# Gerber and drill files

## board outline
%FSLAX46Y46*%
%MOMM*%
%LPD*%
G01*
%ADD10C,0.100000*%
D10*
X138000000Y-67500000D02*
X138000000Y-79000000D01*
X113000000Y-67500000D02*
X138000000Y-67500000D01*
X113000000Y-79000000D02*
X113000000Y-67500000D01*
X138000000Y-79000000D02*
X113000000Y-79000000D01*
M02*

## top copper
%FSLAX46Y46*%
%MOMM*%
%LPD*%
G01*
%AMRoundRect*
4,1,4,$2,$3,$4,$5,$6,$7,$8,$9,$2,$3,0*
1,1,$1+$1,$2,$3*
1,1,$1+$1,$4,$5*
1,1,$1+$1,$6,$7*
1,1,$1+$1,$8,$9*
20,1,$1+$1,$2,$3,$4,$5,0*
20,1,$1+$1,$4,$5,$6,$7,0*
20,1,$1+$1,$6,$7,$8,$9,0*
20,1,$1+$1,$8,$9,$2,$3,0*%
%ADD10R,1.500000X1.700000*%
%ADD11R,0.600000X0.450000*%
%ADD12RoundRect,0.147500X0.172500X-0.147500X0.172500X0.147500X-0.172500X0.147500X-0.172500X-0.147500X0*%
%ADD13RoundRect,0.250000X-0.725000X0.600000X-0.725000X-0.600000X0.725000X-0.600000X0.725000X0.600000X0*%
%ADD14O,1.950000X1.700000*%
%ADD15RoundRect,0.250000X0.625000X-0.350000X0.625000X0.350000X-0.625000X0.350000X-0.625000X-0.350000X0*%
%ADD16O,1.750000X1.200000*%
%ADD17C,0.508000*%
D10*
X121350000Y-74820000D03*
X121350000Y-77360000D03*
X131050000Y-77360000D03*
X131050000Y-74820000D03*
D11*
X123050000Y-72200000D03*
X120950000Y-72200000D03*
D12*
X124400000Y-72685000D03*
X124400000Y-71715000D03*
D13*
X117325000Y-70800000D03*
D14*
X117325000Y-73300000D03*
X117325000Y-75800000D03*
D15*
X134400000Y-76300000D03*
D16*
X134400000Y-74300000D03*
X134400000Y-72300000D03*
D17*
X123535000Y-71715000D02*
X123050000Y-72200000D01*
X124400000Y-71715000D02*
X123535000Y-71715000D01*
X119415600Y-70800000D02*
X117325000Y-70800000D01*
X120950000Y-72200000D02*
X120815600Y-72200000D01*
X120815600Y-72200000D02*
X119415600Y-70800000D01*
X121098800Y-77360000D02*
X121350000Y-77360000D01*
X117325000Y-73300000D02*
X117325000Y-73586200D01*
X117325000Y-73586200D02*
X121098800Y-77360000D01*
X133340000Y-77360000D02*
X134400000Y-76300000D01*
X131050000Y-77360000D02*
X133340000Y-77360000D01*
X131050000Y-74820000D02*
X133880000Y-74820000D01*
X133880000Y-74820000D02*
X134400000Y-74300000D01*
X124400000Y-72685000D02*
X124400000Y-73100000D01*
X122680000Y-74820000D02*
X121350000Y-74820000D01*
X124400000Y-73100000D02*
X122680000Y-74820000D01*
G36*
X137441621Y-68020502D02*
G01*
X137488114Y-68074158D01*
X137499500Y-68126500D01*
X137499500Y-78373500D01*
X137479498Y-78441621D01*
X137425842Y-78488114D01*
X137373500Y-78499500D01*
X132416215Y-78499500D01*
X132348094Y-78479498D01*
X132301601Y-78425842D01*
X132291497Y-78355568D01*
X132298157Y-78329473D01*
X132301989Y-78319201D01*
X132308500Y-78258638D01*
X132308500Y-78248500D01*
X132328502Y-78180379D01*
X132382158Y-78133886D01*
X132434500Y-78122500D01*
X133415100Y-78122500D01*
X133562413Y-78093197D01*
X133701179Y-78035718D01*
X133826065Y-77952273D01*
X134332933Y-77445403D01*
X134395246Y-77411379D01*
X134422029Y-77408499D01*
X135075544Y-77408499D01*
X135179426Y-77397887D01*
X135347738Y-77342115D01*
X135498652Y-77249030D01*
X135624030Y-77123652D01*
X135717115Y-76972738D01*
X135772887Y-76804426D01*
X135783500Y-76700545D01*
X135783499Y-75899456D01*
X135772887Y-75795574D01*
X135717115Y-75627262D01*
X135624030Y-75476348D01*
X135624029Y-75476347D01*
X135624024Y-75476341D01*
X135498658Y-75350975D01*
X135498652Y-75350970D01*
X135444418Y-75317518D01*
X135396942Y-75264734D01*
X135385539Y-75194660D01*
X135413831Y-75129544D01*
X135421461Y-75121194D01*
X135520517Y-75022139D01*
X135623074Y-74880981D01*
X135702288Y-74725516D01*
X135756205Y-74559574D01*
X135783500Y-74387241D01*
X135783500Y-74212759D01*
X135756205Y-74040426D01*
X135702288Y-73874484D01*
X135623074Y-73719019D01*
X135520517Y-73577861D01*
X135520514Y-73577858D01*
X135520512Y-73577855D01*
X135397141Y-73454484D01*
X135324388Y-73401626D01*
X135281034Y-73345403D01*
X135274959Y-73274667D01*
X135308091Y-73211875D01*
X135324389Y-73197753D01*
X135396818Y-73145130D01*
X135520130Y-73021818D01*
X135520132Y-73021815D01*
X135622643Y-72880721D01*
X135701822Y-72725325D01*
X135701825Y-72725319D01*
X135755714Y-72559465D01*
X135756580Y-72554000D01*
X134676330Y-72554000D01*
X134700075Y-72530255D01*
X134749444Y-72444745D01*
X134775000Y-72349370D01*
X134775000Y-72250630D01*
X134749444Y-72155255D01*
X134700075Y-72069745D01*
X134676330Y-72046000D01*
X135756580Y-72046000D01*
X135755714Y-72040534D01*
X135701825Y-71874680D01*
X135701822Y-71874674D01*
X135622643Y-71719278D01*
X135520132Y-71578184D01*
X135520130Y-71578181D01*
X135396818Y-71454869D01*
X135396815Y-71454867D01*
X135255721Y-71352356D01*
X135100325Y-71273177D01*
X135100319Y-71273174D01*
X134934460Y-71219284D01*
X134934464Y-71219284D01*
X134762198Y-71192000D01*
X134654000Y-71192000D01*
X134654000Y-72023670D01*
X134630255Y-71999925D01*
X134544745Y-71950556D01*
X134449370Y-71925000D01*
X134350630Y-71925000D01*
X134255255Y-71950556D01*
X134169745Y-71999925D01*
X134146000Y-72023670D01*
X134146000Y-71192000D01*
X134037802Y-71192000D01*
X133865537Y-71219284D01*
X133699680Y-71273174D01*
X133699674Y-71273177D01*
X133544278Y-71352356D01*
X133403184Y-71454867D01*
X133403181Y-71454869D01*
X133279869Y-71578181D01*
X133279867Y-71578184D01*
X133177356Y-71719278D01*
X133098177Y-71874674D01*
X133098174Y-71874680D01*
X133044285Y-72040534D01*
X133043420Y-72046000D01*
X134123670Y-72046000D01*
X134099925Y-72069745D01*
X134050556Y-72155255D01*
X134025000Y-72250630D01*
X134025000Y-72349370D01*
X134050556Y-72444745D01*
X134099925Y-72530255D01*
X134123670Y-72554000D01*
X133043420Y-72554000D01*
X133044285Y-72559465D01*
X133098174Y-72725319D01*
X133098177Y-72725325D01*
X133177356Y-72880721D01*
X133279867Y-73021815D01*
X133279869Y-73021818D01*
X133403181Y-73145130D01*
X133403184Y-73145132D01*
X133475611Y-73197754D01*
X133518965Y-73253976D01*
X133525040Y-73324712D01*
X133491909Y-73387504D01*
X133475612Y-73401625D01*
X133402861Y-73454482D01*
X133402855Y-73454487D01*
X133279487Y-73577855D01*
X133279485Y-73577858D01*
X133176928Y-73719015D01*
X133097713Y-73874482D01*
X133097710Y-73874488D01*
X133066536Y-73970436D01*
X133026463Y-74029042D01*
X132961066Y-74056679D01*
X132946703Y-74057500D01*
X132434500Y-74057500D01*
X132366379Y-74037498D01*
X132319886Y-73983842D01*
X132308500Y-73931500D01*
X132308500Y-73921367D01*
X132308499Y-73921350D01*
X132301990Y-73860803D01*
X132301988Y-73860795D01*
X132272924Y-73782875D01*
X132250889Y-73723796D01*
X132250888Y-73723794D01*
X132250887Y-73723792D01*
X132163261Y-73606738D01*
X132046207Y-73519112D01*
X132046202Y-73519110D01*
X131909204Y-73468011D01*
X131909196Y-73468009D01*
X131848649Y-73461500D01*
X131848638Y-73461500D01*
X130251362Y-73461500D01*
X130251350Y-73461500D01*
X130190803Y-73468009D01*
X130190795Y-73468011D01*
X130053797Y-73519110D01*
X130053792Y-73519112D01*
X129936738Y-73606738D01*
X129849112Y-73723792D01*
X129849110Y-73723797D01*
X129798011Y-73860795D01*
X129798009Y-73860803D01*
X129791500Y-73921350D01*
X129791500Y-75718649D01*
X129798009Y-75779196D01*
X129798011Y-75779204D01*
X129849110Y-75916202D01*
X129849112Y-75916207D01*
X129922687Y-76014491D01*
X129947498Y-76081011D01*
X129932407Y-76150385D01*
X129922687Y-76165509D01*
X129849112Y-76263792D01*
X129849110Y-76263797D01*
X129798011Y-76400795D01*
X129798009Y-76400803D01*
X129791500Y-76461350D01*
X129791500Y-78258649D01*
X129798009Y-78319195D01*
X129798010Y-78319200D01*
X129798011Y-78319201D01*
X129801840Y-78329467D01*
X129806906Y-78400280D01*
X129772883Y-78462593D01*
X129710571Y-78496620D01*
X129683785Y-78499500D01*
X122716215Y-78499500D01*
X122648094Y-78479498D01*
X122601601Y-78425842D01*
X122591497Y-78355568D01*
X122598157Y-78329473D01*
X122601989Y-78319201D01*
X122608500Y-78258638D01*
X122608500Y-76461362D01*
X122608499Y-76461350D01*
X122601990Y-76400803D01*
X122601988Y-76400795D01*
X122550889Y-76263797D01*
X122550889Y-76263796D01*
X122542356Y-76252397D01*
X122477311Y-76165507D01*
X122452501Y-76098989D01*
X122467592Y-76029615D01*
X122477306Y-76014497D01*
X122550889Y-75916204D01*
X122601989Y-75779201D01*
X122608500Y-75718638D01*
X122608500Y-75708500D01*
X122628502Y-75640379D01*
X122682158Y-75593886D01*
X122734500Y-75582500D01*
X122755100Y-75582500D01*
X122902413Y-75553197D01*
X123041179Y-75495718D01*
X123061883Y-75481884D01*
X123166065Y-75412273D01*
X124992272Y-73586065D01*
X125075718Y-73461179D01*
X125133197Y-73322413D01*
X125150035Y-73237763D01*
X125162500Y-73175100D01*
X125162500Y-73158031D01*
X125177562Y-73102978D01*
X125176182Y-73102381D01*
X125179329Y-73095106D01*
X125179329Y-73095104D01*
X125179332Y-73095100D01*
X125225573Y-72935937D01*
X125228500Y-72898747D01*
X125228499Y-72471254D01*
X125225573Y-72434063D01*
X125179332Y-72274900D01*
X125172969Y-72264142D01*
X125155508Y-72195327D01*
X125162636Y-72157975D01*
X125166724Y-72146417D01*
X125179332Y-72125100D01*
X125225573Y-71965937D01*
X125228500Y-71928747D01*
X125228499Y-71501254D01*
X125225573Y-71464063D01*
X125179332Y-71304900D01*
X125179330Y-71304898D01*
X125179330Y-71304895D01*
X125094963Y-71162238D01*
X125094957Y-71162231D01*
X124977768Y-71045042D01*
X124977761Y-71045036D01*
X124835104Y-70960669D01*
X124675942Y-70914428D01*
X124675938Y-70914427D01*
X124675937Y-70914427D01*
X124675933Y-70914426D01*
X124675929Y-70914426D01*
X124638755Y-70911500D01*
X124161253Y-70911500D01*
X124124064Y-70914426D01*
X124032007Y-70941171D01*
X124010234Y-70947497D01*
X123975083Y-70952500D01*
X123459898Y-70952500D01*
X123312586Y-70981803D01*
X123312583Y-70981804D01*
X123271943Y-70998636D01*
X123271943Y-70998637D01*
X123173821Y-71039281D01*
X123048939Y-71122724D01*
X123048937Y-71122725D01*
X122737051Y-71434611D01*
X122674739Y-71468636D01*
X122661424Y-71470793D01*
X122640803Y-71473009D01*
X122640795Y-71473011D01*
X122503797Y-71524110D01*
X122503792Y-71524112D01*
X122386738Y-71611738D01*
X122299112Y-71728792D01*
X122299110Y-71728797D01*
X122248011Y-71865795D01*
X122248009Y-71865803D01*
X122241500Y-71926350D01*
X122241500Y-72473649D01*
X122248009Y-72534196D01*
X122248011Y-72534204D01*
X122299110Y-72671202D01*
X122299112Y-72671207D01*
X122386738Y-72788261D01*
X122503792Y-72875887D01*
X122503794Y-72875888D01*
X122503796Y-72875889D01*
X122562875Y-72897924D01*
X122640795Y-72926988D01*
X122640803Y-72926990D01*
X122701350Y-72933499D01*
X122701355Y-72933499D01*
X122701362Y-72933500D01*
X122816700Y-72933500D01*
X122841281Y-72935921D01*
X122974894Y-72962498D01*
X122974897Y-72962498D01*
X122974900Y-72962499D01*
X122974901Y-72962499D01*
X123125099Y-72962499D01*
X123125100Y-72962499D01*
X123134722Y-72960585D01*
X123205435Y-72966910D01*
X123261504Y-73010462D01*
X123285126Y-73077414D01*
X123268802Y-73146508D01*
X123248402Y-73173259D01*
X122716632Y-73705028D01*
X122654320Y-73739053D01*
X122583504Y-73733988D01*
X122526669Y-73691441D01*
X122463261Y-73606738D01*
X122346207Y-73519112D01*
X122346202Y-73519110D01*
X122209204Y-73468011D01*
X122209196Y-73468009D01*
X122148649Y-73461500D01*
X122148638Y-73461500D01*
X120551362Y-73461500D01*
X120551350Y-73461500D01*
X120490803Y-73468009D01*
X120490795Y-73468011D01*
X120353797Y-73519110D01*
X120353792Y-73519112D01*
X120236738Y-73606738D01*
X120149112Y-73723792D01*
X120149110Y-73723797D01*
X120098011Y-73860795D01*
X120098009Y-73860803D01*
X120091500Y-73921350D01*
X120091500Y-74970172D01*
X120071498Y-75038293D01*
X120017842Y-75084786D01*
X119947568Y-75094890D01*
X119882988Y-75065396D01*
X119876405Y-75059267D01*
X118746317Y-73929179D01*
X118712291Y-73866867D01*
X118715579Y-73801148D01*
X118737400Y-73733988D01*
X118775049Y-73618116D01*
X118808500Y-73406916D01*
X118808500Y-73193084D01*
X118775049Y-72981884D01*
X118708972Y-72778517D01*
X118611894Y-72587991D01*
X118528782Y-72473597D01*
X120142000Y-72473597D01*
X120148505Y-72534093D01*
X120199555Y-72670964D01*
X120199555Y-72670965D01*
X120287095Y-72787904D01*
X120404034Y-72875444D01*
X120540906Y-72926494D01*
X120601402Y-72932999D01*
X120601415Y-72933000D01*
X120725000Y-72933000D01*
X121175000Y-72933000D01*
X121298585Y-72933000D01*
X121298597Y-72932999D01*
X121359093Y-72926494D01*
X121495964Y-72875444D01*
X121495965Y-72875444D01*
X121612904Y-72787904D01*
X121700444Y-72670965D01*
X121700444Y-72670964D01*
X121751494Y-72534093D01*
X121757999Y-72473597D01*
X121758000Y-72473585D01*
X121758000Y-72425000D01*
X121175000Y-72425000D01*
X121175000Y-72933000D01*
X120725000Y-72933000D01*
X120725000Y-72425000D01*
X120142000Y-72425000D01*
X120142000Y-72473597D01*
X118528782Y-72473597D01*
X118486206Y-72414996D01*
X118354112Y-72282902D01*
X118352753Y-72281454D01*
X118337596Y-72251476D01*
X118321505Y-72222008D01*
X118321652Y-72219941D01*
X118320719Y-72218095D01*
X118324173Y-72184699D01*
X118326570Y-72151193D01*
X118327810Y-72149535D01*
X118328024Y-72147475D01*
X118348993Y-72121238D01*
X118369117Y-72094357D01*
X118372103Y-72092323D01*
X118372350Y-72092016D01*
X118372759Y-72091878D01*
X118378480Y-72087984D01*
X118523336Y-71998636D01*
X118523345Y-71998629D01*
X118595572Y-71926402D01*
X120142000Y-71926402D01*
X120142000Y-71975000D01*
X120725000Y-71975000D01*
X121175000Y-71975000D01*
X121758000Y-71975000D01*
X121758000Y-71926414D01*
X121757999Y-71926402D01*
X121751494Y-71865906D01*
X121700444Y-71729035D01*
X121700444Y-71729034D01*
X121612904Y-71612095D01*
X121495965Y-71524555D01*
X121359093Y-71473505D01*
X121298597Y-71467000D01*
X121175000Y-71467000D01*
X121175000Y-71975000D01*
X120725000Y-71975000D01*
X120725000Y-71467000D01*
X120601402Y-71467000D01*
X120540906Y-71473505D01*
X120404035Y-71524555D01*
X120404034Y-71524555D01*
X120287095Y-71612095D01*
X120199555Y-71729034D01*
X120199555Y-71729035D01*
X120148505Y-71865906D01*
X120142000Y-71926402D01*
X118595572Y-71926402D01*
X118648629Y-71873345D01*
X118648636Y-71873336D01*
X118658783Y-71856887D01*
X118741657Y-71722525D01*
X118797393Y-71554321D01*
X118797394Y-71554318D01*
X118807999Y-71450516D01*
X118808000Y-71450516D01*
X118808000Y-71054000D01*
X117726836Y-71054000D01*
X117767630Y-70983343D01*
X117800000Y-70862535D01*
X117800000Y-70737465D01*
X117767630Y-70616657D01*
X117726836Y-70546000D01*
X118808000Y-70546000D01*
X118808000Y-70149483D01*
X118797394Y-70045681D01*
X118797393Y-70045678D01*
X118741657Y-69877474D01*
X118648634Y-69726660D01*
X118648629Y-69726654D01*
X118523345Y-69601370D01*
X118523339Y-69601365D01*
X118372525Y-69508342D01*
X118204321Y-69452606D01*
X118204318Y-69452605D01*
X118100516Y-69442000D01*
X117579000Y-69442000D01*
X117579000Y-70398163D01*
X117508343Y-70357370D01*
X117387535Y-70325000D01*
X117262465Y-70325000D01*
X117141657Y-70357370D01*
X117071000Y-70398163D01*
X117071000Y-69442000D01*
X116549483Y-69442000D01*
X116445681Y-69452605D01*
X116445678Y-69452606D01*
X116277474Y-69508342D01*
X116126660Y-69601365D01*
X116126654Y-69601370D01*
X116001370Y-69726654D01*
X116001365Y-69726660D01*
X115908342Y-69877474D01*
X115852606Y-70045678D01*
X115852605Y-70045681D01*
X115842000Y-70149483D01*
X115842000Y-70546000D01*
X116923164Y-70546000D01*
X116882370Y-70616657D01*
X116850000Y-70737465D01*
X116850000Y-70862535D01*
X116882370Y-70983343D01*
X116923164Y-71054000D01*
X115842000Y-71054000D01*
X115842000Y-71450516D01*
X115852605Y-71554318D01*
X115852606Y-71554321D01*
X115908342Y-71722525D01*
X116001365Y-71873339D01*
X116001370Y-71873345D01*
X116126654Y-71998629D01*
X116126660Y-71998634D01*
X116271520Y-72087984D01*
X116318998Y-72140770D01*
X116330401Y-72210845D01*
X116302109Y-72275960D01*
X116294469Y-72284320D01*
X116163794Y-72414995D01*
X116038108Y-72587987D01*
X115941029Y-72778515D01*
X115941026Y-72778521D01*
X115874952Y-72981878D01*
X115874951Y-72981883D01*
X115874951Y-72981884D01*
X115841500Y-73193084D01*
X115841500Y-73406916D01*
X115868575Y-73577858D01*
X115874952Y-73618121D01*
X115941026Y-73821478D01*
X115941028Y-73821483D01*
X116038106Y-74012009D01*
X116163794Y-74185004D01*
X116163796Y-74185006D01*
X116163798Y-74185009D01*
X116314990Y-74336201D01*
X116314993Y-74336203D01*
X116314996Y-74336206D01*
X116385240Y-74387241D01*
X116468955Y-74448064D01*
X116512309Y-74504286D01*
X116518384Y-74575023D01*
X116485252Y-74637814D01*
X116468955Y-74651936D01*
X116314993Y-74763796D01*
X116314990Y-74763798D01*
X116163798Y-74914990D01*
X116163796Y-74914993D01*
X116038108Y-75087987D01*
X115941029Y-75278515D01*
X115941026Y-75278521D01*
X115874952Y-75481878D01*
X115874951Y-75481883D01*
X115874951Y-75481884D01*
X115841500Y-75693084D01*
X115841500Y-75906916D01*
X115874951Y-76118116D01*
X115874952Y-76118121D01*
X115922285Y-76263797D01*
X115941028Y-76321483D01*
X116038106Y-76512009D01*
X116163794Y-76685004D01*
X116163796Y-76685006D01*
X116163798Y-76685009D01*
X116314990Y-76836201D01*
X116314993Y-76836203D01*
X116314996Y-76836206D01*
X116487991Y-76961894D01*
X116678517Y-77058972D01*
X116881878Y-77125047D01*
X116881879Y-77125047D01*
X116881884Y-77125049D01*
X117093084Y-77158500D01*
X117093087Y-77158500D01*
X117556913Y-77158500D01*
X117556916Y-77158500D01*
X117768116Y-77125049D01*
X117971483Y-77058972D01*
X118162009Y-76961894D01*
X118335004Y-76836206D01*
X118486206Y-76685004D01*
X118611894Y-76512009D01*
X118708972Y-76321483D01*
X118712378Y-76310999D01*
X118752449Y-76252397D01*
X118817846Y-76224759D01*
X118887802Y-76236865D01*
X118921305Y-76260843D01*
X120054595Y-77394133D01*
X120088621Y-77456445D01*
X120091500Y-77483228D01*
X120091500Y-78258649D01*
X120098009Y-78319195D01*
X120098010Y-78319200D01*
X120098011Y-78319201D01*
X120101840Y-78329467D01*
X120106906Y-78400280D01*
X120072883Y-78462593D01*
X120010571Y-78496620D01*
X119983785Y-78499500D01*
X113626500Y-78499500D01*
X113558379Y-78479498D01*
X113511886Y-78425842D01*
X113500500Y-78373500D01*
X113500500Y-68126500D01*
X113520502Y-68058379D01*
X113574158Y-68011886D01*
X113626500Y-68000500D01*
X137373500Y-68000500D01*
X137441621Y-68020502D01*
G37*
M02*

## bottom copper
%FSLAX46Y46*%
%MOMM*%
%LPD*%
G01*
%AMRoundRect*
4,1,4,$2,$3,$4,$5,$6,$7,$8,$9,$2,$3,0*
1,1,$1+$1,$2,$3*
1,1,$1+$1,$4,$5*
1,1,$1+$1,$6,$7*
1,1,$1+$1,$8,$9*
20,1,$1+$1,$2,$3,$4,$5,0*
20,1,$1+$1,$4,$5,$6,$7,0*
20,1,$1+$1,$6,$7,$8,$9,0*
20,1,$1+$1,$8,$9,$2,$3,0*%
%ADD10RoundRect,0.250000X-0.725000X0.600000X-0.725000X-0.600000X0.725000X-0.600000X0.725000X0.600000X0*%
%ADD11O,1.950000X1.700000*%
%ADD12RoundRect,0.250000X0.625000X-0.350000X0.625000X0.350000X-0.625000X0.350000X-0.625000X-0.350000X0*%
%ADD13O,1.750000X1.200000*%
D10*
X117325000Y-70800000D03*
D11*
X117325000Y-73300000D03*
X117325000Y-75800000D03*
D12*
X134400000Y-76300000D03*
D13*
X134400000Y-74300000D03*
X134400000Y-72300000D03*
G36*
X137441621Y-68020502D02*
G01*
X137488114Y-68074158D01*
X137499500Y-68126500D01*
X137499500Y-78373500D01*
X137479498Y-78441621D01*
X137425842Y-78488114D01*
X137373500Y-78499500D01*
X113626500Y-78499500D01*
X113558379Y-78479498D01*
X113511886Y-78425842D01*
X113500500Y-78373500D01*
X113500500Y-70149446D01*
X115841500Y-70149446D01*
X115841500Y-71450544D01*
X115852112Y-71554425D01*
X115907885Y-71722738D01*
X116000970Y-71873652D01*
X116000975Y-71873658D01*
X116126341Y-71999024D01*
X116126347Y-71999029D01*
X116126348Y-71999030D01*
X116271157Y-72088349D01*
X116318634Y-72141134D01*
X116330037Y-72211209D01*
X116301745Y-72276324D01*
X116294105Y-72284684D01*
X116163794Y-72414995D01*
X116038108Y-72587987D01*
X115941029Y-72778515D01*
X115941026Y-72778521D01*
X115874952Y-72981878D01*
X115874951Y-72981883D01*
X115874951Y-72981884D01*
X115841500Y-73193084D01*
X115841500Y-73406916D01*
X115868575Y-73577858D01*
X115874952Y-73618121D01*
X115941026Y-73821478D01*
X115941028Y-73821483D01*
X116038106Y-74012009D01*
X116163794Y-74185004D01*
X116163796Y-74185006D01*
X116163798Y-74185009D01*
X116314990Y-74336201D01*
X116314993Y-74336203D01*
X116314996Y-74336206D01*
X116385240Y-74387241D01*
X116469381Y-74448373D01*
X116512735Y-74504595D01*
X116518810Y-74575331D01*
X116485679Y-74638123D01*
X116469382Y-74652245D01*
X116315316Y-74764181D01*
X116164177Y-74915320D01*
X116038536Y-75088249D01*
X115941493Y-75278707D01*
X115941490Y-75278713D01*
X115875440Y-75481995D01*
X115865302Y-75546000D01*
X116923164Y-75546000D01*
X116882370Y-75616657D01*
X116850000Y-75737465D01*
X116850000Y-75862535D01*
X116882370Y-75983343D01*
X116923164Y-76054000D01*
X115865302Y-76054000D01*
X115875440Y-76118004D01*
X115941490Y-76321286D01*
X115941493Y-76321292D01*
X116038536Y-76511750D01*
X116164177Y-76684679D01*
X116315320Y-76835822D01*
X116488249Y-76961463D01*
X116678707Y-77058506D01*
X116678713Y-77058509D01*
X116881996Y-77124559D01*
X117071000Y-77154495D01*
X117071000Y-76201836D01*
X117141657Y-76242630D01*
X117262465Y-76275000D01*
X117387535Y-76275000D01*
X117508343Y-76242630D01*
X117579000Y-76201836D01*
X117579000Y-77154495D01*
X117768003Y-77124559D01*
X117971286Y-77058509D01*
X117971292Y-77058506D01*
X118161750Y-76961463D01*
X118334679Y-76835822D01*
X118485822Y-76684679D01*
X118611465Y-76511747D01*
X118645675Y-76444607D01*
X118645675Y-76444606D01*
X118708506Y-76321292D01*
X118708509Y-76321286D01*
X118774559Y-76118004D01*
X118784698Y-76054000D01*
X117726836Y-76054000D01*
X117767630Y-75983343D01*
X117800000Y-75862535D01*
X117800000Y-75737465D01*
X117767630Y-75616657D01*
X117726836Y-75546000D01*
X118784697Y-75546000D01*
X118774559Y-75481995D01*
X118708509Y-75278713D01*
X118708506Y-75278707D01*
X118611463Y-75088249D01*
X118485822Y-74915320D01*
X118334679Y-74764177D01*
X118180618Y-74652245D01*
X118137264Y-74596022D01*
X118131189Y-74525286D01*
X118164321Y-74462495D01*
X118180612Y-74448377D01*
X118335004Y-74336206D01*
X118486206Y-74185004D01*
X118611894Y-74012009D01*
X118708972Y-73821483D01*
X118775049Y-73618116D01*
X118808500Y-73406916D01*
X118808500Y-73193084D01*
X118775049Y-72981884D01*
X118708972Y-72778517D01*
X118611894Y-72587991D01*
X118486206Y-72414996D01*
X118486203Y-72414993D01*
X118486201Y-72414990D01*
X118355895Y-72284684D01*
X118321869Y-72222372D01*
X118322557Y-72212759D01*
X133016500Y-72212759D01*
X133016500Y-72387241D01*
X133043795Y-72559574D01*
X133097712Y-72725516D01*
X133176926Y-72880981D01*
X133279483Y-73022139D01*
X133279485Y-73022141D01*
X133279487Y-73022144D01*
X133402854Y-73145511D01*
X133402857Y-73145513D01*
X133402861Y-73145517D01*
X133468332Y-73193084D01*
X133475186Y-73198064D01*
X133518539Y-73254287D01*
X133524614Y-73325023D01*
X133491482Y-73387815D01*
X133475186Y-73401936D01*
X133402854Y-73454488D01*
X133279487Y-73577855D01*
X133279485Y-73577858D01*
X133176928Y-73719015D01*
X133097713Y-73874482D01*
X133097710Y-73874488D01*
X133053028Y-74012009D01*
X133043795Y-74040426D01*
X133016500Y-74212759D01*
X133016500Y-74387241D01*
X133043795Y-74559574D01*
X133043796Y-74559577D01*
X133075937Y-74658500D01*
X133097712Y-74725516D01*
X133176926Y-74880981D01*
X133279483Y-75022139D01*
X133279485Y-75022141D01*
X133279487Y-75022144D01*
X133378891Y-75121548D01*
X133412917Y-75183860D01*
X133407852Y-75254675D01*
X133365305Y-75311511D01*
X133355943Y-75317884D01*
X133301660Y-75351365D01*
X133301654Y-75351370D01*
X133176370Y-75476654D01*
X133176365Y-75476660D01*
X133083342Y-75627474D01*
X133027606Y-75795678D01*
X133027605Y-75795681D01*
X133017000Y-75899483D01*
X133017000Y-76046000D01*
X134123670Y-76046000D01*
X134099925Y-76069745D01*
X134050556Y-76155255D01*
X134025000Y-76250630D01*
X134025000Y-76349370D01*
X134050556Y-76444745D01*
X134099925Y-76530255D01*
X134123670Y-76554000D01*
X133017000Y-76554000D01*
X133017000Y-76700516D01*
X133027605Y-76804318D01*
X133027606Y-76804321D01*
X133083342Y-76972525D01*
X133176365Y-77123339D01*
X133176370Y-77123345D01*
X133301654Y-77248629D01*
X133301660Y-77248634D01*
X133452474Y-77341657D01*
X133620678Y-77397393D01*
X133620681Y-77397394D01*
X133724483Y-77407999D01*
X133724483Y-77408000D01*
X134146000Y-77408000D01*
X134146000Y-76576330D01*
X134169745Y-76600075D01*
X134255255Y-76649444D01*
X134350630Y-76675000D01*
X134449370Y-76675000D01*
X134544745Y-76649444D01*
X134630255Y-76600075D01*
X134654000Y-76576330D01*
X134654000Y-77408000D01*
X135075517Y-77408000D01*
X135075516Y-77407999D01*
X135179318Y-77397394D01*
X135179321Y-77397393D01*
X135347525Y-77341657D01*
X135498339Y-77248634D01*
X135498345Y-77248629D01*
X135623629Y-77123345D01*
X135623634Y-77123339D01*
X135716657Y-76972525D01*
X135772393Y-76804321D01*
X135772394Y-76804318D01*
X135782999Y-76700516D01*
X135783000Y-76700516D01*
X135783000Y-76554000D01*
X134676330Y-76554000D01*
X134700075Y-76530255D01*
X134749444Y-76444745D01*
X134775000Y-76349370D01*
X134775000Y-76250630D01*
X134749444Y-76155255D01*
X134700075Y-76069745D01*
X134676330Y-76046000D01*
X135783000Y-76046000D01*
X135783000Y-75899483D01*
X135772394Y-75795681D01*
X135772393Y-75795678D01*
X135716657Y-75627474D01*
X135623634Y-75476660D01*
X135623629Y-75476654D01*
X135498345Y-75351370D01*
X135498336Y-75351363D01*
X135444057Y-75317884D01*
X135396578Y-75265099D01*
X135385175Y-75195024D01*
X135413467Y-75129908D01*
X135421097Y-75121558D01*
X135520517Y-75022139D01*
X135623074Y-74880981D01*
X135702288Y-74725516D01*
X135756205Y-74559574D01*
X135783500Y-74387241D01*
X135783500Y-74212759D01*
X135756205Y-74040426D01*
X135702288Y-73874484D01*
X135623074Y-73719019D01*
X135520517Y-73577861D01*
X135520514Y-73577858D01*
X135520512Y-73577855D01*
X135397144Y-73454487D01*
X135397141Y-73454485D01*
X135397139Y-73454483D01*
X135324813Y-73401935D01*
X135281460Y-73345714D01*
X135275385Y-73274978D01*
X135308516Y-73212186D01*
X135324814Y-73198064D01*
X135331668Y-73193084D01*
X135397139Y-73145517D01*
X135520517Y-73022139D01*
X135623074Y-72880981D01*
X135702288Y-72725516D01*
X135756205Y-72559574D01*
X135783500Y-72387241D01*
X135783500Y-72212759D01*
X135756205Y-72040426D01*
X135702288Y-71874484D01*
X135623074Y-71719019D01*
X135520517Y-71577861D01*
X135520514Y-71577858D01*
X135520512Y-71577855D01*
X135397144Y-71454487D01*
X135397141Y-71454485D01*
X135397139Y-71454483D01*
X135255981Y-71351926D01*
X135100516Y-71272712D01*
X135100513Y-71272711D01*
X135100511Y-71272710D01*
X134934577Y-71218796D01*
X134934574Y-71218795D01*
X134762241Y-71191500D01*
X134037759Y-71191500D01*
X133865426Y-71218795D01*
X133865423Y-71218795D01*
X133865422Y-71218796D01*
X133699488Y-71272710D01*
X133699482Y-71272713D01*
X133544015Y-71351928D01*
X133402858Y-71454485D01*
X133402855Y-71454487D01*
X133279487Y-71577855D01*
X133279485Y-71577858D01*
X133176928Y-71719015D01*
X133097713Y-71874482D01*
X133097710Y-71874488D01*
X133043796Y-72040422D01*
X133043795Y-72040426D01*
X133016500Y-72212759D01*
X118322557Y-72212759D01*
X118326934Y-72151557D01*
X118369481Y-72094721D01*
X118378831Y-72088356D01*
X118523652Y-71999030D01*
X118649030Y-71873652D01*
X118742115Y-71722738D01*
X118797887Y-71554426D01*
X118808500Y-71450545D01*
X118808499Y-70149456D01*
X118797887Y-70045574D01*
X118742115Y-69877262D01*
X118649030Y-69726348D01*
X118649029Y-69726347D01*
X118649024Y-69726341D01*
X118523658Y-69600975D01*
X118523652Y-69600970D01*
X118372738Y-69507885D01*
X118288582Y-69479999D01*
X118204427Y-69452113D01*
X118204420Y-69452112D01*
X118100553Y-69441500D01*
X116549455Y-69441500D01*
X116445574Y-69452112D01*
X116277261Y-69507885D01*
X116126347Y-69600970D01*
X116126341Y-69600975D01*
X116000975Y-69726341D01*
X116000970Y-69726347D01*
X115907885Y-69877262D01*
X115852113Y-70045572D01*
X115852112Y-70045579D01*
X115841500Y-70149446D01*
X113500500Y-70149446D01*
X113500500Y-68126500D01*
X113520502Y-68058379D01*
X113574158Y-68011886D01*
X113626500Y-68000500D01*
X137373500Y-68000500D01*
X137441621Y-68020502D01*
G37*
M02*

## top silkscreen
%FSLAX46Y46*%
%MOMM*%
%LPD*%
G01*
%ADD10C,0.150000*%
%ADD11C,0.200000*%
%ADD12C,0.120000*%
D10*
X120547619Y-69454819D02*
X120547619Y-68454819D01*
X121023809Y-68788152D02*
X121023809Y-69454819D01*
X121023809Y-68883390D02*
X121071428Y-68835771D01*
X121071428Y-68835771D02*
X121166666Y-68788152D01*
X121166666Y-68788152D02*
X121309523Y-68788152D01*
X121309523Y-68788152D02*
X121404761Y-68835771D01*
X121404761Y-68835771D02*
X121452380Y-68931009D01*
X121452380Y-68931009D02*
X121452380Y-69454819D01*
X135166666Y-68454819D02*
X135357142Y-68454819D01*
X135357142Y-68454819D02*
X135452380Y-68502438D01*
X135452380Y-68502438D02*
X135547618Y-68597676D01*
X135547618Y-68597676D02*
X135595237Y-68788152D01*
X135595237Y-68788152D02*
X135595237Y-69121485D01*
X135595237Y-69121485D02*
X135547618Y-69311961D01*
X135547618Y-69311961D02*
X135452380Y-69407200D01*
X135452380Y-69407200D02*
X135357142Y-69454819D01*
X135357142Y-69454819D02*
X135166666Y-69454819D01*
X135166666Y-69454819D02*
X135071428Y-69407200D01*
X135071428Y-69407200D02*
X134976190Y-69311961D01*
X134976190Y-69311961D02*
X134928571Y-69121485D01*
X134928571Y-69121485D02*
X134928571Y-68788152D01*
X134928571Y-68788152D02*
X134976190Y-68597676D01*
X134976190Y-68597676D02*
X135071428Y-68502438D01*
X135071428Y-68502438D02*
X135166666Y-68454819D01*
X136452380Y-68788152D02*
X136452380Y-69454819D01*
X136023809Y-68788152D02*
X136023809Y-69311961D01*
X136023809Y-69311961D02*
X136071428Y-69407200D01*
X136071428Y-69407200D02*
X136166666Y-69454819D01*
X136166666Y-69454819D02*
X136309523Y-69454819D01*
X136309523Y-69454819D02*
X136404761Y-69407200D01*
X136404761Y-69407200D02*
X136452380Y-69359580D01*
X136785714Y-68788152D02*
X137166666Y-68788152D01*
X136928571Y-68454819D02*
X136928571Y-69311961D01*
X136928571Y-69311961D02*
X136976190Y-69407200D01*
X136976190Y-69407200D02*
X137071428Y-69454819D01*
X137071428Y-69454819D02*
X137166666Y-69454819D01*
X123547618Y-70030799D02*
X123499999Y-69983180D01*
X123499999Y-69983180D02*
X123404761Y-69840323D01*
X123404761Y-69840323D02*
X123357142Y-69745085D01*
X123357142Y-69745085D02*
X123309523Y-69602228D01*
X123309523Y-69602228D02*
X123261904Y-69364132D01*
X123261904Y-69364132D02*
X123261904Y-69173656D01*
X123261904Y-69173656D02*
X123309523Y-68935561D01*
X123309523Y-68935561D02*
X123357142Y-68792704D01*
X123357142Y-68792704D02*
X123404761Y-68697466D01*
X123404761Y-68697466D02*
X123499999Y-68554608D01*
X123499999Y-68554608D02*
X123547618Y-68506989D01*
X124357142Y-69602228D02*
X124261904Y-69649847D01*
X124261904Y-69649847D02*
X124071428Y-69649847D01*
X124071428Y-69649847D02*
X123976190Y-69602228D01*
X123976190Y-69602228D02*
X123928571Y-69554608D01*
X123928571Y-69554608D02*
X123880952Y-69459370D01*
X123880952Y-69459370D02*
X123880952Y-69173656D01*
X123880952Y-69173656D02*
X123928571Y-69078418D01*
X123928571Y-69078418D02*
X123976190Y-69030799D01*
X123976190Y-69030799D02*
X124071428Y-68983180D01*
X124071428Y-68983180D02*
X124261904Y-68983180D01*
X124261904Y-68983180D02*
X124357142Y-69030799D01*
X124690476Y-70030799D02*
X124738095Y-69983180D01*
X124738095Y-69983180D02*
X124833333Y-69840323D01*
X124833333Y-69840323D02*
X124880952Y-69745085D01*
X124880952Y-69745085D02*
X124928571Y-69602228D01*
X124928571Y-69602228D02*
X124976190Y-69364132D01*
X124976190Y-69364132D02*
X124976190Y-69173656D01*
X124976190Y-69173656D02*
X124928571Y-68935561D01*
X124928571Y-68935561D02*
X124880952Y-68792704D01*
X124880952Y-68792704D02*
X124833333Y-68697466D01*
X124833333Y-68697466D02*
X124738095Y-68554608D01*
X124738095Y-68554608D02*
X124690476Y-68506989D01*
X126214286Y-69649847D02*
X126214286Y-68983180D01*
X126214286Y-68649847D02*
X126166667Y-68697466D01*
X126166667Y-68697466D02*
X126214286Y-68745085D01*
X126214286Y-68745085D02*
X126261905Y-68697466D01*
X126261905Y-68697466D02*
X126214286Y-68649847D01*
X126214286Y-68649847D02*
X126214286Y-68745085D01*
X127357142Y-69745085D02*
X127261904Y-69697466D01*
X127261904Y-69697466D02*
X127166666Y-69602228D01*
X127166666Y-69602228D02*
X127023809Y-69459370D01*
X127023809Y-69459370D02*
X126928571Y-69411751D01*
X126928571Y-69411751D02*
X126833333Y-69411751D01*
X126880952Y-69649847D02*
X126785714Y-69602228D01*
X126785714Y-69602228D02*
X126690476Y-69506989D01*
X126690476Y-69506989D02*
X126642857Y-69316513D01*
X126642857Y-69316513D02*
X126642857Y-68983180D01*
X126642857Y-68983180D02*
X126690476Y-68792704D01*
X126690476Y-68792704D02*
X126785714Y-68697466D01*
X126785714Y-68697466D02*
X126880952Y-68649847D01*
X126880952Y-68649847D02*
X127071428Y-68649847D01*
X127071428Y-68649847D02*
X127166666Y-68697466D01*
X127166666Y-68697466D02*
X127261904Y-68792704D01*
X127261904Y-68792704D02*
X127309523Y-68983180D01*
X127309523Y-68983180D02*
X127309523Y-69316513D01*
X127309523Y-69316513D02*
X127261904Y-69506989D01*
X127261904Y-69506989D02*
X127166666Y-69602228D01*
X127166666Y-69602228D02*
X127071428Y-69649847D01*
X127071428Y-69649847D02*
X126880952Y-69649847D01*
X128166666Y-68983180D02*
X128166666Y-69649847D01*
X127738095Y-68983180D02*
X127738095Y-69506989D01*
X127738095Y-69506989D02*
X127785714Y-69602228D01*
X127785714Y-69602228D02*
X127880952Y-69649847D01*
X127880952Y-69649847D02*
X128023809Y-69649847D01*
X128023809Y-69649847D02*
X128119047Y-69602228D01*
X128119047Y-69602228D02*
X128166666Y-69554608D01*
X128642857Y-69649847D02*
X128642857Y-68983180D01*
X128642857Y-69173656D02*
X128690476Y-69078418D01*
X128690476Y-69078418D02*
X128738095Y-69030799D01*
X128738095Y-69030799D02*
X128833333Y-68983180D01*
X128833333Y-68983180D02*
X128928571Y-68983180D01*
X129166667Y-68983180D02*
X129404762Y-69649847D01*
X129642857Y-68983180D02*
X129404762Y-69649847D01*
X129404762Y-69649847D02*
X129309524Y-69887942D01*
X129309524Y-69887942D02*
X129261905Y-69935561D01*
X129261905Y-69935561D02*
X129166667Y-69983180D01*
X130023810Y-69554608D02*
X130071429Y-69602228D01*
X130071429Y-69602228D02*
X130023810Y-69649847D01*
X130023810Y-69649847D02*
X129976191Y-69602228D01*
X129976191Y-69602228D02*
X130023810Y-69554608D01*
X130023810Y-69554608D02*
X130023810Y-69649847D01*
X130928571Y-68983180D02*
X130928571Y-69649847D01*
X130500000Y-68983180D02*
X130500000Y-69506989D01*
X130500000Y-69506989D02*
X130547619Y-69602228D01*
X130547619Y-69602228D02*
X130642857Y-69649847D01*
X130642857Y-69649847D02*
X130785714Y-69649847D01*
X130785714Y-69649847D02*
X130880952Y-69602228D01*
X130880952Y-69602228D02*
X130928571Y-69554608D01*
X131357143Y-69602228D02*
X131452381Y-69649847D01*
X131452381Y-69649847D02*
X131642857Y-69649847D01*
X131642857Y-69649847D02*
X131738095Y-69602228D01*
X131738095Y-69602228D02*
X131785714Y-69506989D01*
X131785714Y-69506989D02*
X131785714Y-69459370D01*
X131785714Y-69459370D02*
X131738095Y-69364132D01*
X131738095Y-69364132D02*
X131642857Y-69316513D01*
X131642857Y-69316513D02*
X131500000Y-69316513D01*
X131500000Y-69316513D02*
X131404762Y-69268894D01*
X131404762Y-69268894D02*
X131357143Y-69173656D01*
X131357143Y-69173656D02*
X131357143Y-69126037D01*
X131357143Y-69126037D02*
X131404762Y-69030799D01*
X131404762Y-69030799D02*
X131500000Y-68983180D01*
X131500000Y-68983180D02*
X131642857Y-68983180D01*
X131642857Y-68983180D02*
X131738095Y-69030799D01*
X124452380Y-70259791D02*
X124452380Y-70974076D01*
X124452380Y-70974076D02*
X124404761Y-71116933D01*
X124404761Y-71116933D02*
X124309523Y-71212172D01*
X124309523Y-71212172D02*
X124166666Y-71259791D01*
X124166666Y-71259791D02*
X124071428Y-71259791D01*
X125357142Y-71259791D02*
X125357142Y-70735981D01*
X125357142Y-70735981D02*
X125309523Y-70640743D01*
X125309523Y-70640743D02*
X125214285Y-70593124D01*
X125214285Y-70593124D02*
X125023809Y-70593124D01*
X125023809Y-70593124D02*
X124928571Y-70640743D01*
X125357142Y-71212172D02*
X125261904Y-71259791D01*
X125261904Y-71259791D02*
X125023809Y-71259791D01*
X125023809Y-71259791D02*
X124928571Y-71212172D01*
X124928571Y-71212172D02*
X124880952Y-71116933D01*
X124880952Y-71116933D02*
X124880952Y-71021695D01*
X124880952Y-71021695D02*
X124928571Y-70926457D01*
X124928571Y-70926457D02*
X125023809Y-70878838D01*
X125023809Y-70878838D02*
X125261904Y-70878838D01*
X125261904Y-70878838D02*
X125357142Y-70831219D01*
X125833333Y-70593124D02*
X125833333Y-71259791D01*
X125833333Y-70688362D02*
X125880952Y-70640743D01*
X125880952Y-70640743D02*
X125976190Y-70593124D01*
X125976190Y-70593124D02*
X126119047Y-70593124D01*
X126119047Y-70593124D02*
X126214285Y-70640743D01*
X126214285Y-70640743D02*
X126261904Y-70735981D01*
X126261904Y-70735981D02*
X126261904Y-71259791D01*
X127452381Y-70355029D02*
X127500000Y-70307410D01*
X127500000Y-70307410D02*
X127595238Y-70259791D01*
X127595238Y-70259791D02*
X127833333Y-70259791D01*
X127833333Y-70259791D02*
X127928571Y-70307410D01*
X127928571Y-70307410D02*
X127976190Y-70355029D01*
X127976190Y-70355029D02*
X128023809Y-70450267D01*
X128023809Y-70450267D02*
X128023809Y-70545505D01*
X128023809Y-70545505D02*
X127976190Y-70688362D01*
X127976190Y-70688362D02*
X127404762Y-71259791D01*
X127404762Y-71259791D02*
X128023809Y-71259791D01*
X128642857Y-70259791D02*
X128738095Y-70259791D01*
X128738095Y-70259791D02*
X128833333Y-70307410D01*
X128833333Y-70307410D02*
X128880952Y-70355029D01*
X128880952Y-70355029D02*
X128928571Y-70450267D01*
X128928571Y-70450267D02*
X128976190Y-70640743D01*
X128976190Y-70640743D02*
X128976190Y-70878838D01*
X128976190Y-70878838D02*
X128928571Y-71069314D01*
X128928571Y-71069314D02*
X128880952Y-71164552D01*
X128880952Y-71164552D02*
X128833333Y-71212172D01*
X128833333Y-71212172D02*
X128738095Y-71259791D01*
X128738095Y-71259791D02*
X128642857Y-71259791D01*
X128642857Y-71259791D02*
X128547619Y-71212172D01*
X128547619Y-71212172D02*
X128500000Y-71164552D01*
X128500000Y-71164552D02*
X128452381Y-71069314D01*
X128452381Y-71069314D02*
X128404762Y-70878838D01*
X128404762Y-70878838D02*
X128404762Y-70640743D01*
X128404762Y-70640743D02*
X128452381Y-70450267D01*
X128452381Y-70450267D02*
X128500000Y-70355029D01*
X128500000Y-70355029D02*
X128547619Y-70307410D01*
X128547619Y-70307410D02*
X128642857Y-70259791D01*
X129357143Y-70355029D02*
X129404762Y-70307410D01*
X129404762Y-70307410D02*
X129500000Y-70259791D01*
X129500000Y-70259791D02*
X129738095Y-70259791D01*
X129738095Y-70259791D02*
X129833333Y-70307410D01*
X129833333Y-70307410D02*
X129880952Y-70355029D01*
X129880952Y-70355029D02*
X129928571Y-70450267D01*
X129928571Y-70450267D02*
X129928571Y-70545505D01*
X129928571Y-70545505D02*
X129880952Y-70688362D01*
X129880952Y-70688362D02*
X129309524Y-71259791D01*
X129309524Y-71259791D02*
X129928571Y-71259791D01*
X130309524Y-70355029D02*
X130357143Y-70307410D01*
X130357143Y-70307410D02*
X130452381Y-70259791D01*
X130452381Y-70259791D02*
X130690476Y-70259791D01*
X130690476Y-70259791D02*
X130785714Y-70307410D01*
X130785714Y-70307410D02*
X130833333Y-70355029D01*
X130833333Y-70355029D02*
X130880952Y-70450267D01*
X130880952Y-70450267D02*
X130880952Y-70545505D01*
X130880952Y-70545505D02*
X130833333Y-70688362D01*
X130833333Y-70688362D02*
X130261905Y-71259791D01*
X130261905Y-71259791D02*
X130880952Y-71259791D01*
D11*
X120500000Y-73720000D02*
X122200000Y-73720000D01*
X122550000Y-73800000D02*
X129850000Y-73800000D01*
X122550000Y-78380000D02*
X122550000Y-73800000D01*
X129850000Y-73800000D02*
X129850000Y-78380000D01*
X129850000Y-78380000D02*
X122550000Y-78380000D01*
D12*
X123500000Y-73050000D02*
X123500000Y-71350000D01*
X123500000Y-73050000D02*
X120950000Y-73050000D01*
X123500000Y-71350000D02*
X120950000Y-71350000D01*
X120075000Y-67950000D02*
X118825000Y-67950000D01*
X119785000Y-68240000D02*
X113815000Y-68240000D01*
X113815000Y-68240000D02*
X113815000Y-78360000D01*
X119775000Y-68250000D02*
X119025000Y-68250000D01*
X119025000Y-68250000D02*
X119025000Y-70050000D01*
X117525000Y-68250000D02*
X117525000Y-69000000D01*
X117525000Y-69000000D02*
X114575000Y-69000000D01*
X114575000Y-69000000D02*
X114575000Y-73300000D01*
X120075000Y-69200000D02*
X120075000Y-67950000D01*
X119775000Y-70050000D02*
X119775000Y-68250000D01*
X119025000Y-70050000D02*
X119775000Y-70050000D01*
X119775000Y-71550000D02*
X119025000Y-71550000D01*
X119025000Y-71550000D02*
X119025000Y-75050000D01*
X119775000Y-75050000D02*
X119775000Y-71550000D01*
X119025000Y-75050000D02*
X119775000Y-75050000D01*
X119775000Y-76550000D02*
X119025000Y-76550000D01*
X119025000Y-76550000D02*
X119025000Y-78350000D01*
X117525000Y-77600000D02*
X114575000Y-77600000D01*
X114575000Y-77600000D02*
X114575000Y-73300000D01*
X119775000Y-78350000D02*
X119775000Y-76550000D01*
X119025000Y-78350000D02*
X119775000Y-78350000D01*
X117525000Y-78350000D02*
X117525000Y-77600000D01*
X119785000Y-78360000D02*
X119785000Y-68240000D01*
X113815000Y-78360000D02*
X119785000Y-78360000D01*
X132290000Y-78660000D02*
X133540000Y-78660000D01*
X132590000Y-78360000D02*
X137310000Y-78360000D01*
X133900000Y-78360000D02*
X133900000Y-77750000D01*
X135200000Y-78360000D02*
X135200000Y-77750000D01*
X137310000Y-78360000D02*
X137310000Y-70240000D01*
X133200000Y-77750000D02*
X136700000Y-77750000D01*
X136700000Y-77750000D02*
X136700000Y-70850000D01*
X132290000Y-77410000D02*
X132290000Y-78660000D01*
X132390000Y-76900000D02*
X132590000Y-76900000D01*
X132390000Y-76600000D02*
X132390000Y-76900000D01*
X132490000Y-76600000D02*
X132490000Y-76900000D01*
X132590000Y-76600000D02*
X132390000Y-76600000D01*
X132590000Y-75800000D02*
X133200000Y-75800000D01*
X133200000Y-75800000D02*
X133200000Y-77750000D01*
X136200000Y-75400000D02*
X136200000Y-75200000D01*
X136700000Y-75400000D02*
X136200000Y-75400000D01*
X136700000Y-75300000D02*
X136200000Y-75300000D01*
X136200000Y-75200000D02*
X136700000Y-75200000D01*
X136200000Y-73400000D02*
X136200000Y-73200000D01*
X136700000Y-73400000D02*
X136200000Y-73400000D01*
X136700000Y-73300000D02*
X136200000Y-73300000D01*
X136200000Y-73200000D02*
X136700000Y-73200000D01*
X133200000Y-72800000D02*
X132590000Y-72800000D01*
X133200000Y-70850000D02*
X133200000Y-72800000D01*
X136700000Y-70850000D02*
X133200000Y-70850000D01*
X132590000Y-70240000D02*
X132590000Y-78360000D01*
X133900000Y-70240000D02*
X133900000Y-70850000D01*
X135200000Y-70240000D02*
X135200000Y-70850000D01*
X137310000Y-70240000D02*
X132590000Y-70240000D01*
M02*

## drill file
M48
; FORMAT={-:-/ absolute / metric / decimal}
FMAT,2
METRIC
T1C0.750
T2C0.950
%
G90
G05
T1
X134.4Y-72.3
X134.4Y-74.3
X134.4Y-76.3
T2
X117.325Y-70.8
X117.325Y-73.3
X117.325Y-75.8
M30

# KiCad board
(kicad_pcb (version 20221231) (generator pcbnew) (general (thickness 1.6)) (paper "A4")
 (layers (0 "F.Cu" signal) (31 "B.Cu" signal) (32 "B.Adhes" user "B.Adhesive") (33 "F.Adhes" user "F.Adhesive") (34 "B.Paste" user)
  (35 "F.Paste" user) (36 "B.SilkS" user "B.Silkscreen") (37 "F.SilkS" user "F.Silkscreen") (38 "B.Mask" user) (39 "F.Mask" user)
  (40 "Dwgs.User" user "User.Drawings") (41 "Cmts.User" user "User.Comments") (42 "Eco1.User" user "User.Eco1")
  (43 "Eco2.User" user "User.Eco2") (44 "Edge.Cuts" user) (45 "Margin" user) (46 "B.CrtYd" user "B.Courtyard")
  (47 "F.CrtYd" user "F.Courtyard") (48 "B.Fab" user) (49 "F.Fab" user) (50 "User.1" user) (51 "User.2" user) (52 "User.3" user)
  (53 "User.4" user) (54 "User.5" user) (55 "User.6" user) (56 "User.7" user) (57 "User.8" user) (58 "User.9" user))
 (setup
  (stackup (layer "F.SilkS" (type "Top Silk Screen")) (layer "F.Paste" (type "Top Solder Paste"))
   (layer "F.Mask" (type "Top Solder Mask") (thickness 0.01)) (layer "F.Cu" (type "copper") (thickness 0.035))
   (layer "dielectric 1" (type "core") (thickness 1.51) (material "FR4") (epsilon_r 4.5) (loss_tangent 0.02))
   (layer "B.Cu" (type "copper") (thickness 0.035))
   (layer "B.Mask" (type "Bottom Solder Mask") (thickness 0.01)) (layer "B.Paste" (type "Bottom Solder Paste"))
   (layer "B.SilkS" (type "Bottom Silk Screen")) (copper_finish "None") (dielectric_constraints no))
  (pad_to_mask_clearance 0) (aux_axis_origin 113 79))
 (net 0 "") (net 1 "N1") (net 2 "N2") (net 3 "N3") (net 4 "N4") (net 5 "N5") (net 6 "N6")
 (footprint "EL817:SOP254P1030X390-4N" (layer "F.Cu") (at 126.2 76.09)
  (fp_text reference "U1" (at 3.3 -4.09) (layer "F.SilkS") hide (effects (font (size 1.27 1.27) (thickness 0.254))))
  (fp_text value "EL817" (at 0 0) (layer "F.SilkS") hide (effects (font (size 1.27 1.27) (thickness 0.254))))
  (fp_line (start -5.7 -2.37) (end -4 -2.37) (stroke (width 0.2) (type solid)) (layer "F.SilkS"))
  (fp_line (start -3.65 -2.29) (end 3.65 -2.29) (stroke (width 0.2) (type solid)) (layer "F.SilkS"))
  (fp_line (start -3.65 2.29) (end -3.65 -2.29) (stroke (width 0.2) (type solid)) (layer "F.SilkS"))
  (fp_line (start 3.65 -2.29) (end 3.65 2.29) (stroke (width 0.2) (type solid)) (layer "F.SilkS"))
  (fp_line (start 3.65 2.29) (end -3.65 2.29) (stroke (width 0.2) (type solid)) (layer "F.SilkS"))
  (pad "1" smd rect (at -4.85 -1.27) (size 1.5 1.7) (layers "F.Cu" "F.Paste" "F.Mask") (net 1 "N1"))
  (pad "2" smd rect (at -4.85 1.27) (size 1.5 1.7) (layers "F.Cu" "F.Paste" "F.Mask") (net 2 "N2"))
  (pad "3" smd rect (at 4.85 1.27) (size 1.5 1.7) (layers "F.Cu" "F.Paste" "F.Mask") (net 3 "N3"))
  (pad "4" smd rect (at 4.85 -1.27) (size 1.5 1.7) (layers "F.Cu" "F.Paste" "F.Mask") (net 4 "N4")))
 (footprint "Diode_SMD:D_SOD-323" (layer "F.Cu") (at 122 72.2 180)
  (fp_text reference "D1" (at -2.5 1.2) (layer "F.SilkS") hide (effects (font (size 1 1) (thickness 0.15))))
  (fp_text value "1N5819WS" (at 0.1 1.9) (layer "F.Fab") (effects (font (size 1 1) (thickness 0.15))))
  (fp_line (start -1.5 -0.85) (end -1.5 0.85) (stroke (width 0.12) (type solid)) (layer "F.SilkS"))
  (fp_line (start -1.5 -0.85) (end 1.05 -0.85) (stroke (width 0.12) (type solid)) (layer "F.SilkS"))
  (fp_line (start -1.5 0.85) (end 1.05 0.85) (stroke (width 0.12) (type solid)) (layer "F.SilkS"))
  (pad "1" smd rect locked (at -1.05 0 180) (size 0.6 0.45) (layers "F.Cu" "F.Paste" "F.Mask") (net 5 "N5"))
  (pad "2" smd rect locked (at 1.05 0 180) (size 0.6 0.45) (layers "F.Cu" "F.Paste" "F.Mask") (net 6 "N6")))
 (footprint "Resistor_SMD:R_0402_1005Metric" (layer "F.Cu") (at 124.4 72.2 90)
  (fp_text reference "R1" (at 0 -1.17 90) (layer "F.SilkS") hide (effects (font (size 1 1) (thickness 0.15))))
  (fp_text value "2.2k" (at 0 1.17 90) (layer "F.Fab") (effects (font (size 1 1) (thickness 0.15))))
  (pad "1" smd roundrect locked (at -0.485 0 90) (size 0.59 0.64) (layers "F.Cu" "F.Paste" "F.Mask") (roundrect_rratio 0.25) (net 1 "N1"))
  (pad "2" smd roundrect locked (at 0.485 0 90) (size 0.59 0.64) (layers "F.Cu" "F.Paste" "F.Mask") (roundrect_rratio 0.25) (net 5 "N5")))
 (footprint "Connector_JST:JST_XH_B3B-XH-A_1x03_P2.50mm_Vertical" (layer "F.Cu") (at 117.325 70.8 -90)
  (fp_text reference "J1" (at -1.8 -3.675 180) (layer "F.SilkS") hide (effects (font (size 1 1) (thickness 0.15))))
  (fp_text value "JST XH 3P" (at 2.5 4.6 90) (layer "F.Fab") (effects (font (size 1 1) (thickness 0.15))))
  (fp_line (start -2.85 -2.75) (end -2.85 -1.5) (stroke (width 0.12) (type solid)) (layer "F.SilkS"))
  (fp_line (start -2.56 -2.46) (end -2.56 3.51) (stroke (width 0.12) (type solid)) (layer "F.SilkS"))
  (fp_line (start -2.56 3.51) (end 7.56 3.51) (stroke (width 0.12) (type solid)) (layer "F.SilkS"))
  (fp_line (start -2.55 -2.45) (end -2.55 -1.7) (stroke (width 0.12) (type solid)) (layer "F.SilkS"))
  (fp_line (start -2.55 -1.7) (end -0.75 -1.7) (stroke (width 0.12) (type solid)) (layer "F.SilkS"))
  (fp_line (start -2.55 -0.2) (end -1.8 -0.2) (stroke (width 0.12) (type solid)) (layer "F.SilkS"))
  (fp_line (start -1.8 -0.2) (end -1.8 2.75) (stroke (width 0.12) (type solid)) (layer "F.SilkS"))
  (fp_line (start -1.8 2.75) (end 2.5 2.75) (stroke (width 0.12) (type solid)) (layer "F.SilkS"))
  (fp_line (start -1.6 -2.75) (end -2.85 -2.75) (stroke (width 0.12) (type solid)) (layer "F.SilkS"))
  (fp_line (start -0.75 -2.45) (end -2.55 -2.45) (stroke (width 0.12) (type solid)) (layer "F.SilkS"))
  (fp_line (start -0.75 -1.7) (end -0.75 -2.45) (stroke (width 0.12) (type solid)) (layer "F.SilkS"))
  (fp_line (start 0.75 -2.45) (end 0.75 -1.7) (stroke (width 0.12) (type solid)) (layer "F.SilkS"))
  (fp_line (start 0.75 -1.7) (end 4.25 -1.7) (stroke (width 0.12) (type solid)) (layer "F.SilkS"))
  (fp_line (start 4.25 -2.45) (end 0.75 -2.45) (stroke (width 0.12) (type solid)) (layer "F.SilkS"))
  (fp_line (start 4.25 -1.7) (end 4.25 -2.45) (stroke (width 0.12) (type solid)) (layer "F.SilkS"))
  (fp_line (start 5.75 -2.45) (end 5.75 -1.7) (stroke (width 0.12) (type solid)) (layer "F.SilkS"))
  (fp_line (start 5.75 -1.7) (end 7.55 -1.7) (stroke (width 0.12) (type solid)) (layer "F.SilkS"))
  (fp_line (start 6.8 -0.2) (end 6.8 2.75) (stroke (width 0.12) (type solid)) (layer "F.SilkS"))
  (fp_line (start 6.8 2.75) (end 2.5 2.75) (stroke (width 0.12) (type solid)) (layer "F.SilkS"))
  (fp_line (start 7.55 -2.45) (end 5.75 -2.45) (stroke (width 0.12) (type solid)) (layer "F.SilkS"))
  (fp_line (start 7.55 -1.7) (end 7.55 -2.45) (stroke (width 0.12) (type solid)) (layer "F.SilkS"))
  (fp_line (start 7.55 -0.2) (end 6.8 -0.2) (stroke (width 0.12) (type solid)) (layer "F.SilkS"))
  (fp_line (start 7.56 -2.46) (end -2.56 -2.46) (stroke (width 0.12) (type solid)) (layer "F.SilkS"))
  (fp_line (start 7.56 3.51) (end 7.56 -2.46) (stroke (width 0.12) (type solid)) (layer "F.SilkS"))
  (pad "1" thru_hole roundrect locked (at 0 0 270) (size 1.7 1.95) (drill 0.95) (layers *.Cu *.Mask) (roundrect_rratio 0.1470588235)
   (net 6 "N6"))
  (pad "2" thru_hole oval locked (at 2.5 0 270) (size 1.7 1.95) (drill 0.95) (layers *.Cu *.Mask) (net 2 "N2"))
  (pad "3" thru_hole oval locked (at 5 0 270) (size 1.7 1.95) (drill 0.95) (layers *.Cu *.Mask) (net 3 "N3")))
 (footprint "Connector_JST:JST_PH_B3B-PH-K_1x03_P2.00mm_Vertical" (layer "F.Cu") (at 134.4 76.3 90)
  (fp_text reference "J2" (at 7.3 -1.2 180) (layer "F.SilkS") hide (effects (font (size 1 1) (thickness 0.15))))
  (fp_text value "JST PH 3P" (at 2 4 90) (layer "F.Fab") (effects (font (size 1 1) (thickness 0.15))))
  (fp_line (start -2.36 -2.11) (end -2.36 -0.86) (stroke (width 0.12) (type solid)) (layer "F.SilkS"))
  (fp_line (start -2.06 -1.81) (end -2.06 2.91) (stroke (width 0.12) (type solid)) (layer "F.SilkS"))
  (fp_line (start -2.06 -0.5) (end -1.45 -0.5) (stroke (width 0.12) (type solid)) (layer "F.SilkS"))
  (fp_line (start -2.06 0.8) (end -1.45 0.8) (stroke (width 0.12) (type solid)) (layer "F.SilkS"))
  (fp_line (start -2.06 2.91) (end 6.06 2.91) (stroke (width 0.12) (type solid)) (layer "F.SilkS"))
  (fp_line (start -1.45 -1.2) (end -1.45 2.3) (stroke (width 0.12) (type solid)) (layer "F.SilkS"))
  (fp_line (start -1.45 2.3) (end 5.45 2.3) (stroke (width 0.12) (type solid)) (layer "F.SilkS"))
  (fp_line (start -1.11 -2.11) (end -2.36 -2.11) (stroke (width 0.12) (type solid)) (layer "F.SilkS"))
  (fp_line (start -0.6 -2.01) (end -0.6 -1.81) (stroke (width 0.12) (type solid)) (layer "F.SilkS"))
  (fp_line (start -0.3 -2.01) (end -0.6 -2.01) (stroke (width 0.12) (type solid)) (layer "F.SilkS"))
  (fp_line (start -0.3 -1.91) (end -0.6 -1.91) (stroke (width 0.12) (type solid)) (layer "F.SilkS"))
  (fp_line (start -0.3 -1.81) (end -0.3 -2.01) (stroke (width 0.12) (type solid)) (layer "F.SilkS"))
  (fp_line (start 0.5 -1.81) (end 0.5 -1.2) (stroke (width 0.12) (type solid)) (layer "F.SilkS"))
  (fp_line (start 0.5 -1.2) (end -1.45 -1.2) (stroke (width 0.12) (type solid)) (layer "F.SilkS"))
  (fp_line (start 0.9 1.8) (end 1.1 1.8) (stroke (width 0.12) (type solid)) (layer "F.SilkS"))
  (fp_line (start 0.9 2.3) (end 0.9 1.8) (stroke (width 0.12) (type solid)) (layer "F.SilkS"))
  (fp_line (start 1 2.3) (end 1 1.8) (stroke (width 0.12) (type solid)) (layer "F.SilkS"))
  (fp_line (start 1.1 1.8) (end 1.1 2.3) (stroke (width 0.12) (type solid)) (layer "F.SilkS"))
  (fp_line (start 2.9 1.8) (end 3.1 1.8) (stroke (width 0.12) (type solid)) (layer "F.SilkS"))
  (fp_line (start 2.9 2.3) (end 2.9 1.8) (stroke (width 0.12) (type solid)) (layer "F.SilkS"))
  (fp_line (start 3 2.3) (end 3 1.8) (stroke (width 0.12) (type solid)) (layer "F.SilkS"))
  (fp_line (start 3.1 1.8) (end 3.1 2.3) (stroke (width 0.12) (type solid)) (layer "F.SilkS"))
  (fp_line (start 3.5 -1.2) (end 3.5 -1.81) (stroke (width 0.12) (type solid)) (layer "F.SilkS"))
  (fp_line (start 5.45 -1.2) (end 3.5 -1.2) (stroke (width 0.12) (type solid)) (layer "F.SilkS"))
  (fp_line (start 5.45 2.3) (end 5.45 -1.2) (stroke (width 0.12) (type solid)) (layer "F.SilkS"))
  (fp_line (start 6.06 -1.81) (end -2.06 -1.81) (stroke (width 0.12) (type solid)) (layer "F.SilkS"))
  (fp_line (start 6.06 -0.5) (end 5.45 -0.5) (stroke (width 0.12) (type solid)) (layer "F.SilkS"))
  (fp_line (start 6.06 0.8) (end 5.45 0.8) (stroke (width 0.12) (type solid)) (layer "F.SilkS"))
  (fp_line (start 6.06 2.91) (end 6.06 -1.81) (stroke (width 0.12) (type solid)) (layer "F.SilkS"))
  (pad "1" thru_hole roundrect locked (at 0 0 90) (size 1.2 1.75) (drill 0.75) (layers *.Cu *.Mask) (roundrect_rratio 0.2083333333)
   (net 3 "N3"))
  (pad "2" thru_hole oval locked (at 2 0 90) (size 1.2 1.75) (drill 0.75) (layers *.Cu *.Mask) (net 4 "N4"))
  (pad "3" thru_hole oval locked (at 4 0 90) (size 1.2 1.75) (drill 0.75) (layers *.Cu *.Mask) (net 6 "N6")))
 (gr_line (start 138 67.5) (end 138 79) (stroke (width 0.1) (type solid)) (layer "Edge.Cuts"))
 (gr_line (start 113 67.5) (end 138 67.5) (stroke (width 0.1) (type solid)) (layer "Edge.Cuts"))
 (gr_line (start 113 79) (end 113 67.5) (stroke (width 0.1) (type solid)) (layer "Edge.Cuts"))
 (gr_line (start 138 79) (end 113 79) (stroke (width 0.1) (type solid)) (layer "Edge.Cuts"))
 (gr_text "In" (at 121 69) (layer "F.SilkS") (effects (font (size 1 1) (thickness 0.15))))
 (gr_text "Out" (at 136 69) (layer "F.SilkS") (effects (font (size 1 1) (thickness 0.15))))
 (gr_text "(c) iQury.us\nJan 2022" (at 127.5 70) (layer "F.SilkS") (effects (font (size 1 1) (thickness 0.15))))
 (segment (start 123.535 71.715) (end 123.05 72.2) (width 0.508) (layer "F.Cu") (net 5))
 (segment (start 124.4 71.715) (end 123.535 71.715) (width 0.508) (layer "F.Cu") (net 5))
 (segment (start 119.4156 70.8) (end 117.325 70.8) (width 0.508) (layer "F.Cu") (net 6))
 (segment (start 120.95 72.2) (end 120.8156 72.2) (width 0.508) (layer "F.Cu") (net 6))
 (segment (start 120.8156 72.2) (end 119.4156 70.8) (width 0.508) (layer "F.Cu") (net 6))
 (segment (start 121.0988 77.36) (end 121.35 77.36) (width 0.508) (layer "F.Cu") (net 2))
 (segment (start 117.325 73.3) (end 117.325 73.5862) (width 0.508) (layer "F.Cu") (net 2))
 (segment (start 117.325 73.5862) (end 121.0988 77.36) (width 0.508) (layer "F.Cu") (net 2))
 (segment (start 133.34 77.36) (end 134.4 76.3) (width 0.508) (layer "F.Cu") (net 3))
 (segment (start 131.05 77.36) (end 133.34 77.36) (width 0.508) (layer "F.Cu") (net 3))
 (segment (start 131.05 74.82) (end 133.88 74.82) (width 0.508) (layer "F.Cu") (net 4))
 (segment (start 133.88 74.82) (end 134.4 74.3) (width 0.508) (layer "F.Cu") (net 4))
 (segment (start 124.4 72.685) (end 124.4 73.1) (width 0.508) (layer "F.Cu") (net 1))
 (segment (start 122.68 74.82) (end 121.35 74.82) (width 0.508) (layer "F.Cu") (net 1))
 (segment (start 124.4 73.1) (end 122.68 74.82) (width 0.508) (layer "F.Cu") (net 1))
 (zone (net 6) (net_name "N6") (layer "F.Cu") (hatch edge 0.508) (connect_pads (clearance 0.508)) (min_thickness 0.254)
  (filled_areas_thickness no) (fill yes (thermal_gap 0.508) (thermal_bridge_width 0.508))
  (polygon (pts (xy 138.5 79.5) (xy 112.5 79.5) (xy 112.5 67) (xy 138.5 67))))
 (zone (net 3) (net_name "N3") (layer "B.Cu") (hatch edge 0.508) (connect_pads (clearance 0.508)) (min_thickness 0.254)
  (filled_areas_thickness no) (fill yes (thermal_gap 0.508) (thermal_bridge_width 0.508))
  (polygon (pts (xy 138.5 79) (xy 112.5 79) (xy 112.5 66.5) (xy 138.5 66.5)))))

